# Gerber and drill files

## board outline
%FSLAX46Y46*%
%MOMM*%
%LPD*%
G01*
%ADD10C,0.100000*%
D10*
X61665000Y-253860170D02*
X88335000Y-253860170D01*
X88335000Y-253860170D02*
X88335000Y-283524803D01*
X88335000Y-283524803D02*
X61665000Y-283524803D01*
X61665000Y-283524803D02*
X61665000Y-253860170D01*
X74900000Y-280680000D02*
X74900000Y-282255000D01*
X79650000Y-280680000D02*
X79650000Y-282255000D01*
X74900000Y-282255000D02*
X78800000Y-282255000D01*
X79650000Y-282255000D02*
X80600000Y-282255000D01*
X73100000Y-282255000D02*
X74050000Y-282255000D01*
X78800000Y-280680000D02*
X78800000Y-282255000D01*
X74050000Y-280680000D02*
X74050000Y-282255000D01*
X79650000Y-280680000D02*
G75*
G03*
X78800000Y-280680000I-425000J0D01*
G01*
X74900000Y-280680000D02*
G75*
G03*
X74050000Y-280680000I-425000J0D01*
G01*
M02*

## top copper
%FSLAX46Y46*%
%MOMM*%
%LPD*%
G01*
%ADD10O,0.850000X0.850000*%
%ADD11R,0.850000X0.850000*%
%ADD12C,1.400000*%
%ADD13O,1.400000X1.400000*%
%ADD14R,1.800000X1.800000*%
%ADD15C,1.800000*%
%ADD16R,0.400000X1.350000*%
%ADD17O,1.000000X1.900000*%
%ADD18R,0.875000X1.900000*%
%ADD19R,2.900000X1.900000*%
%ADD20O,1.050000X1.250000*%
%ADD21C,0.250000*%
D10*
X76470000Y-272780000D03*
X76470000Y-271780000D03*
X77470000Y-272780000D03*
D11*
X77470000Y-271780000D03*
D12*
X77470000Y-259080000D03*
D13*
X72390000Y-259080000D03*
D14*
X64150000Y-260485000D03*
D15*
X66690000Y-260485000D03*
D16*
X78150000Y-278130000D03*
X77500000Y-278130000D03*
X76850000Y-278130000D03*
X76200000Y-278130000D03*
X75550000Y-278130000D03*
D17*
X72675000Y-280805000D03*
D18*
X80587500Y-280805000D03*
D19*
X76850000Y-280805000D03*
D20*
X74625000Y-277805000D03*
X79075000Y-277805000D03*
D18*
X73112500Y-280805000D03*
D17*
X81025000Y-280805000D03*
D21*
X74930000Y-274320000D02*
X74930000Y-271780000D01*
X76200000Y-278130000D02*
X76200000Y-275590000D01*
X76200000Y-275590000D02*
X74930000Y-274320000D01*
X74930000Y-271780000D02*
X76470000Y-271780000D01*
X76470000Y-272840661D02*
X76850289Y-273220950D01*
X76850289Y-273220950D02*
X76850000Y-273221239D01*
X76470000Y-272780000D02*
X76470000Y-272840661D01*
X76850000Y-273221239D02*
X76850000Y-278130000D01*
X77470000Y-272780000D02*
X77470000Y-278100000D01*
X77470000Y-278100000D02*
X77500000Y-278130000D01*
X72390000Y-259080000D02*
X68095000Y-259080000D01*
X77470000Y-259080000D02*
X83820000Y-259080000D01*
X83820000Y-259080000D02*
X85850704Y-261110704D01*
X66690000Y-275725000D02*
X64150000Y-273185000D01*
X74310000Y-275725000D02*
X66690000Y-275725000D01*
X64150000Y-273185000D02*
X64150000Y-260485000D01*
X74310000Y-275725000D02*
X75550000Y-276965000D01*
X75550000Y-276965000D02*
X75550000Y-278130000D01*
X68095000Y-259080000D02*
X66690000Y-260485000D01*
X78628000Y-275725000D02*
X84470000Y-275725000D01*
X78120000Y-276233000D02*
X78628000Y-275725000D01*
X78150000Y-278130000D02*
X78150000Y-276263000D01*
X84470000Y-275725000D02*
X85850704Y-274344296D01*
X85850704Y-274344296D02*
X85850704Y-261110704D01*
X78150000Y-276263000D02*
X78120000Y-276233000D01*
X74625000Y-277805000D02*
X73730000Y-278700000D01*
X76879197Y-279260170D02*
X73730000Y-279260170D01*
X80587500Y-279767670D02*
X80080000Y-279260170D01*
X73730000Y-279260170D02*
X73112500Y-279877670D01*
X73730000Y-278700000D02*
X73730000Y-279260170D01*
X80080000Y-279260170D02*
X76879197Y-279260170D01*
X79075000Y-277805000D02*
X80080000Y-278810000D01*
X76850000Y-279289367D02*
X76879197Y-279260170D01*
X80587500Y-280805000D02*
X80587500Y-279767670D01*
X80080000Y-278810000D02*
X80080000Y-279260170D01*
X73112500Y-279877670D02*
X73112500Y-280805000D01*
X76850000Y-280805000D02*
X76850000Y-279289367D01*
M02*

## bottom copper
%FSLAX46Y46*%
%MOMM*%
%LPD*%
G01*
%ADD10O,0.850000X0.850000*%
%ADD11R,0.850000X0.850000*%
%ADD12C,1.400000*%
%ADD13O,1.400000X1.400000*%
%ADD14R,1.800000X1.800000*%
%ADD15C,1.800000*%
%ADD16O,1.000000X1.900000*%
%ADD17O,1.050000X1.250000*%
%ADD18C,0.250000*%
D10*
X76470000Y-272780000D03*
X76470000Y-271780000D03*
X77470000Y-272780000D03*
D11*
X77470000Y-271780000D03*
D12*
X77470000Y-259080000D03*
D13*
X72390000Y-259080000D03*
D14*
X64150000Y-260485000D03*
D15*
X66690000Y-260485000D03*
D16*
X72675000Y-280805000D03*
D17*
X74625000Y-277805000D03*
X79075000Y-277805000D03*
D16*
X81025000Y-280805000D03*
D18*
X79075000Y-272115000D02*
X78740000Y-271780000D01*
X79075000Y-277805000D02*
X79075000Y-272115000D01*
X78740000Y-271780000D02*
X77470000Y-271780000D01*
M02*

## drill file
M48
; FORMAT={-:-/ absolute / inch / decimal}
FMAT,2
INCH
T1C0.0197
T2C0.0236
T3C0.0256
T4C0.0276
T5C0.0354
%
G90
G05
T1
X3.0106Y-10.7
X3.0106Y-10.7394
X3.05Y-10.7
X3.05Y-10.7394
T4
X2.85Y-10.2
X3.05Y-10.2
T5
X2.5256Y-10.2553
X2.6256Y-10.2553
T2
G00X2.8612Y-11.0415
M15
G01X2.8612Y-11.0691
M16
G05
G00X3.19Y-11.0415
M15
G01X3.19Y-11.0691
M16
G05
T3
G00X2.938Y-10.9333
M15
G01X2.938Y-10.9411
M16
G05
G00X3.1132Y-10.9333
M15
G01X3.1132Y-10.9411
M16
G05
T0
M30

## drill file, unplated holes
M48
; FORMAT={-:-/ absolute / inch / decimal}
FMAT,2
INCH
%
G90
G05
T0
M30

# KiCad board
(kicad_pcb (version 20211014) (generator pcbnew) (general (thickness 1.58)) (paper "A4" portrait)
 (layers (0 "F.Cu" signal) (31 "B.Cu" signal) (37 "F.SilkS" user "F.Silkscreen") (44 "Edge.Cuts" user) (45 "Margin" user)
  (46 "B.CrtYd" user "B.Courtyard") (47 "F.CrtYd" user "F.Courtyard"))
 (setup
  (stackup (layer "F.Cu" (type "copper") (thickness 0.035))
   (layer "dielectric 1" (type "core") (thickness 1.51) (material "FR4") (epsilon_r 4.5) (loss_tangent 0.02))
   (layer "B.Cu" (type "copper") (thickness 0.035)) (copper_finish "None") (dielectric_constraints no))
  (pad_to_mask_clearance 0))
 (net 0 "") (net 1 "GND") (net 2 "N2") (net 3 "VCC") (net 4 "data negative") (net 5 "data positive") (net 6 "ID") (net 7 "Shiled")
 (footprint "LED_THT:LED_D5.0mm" (layer "F.Cu") (at 64.15 260.485)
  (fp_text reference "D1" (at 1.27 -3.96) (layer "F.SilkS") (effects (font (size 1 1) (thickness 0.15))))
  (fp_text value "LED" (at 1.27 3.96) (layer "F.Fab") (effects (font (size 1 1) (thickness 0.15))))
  (pad "1" thru_hole rect (at 0 0) (size 1.8 1.8) (drill 0.9) (layers *.Cu *.Mask) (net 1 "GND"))
  (pad "2" thru_hole circle (at 2.54 0) (size 1.8 1.8) (drill 0.9) (layers *.Cu *.Mask) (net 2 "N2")))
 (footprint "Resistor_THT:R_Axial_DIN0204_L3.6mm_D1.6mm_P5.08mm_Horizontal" (layer "F.Cu") (at 77.47 259.08 180)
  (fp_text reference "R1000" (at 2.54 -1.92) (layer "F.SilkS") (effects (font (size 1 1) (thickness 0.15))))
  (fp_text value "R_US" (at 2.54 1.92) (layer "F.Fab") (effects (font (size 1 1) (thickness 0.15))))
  (pad "1" thru_hole circle (at 0 0 180) (size 1.4 1.4) (drill 0.7) (layers *.Cu *.Mask) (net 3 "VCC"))
  (pad "2" thru_hole oval (at 5.08 0 180) (size 1.4 1.4) (drill 0.7) (layers *.Cu *.Mask) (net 2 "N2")))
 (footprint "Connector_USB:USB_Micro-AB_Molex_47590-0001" (layer "F.Cu") (at 76.85 280.805)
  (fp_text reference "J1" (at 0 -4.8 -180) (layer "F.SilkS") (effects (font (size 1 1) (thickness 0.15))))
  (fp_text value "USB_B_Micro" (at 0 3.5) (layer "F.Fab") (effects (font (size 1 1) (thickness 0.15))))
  (fp_line (start -1.95 -0.125) (end -1.95 1.45) (layer "Edge.Cuts") (width 0.1))
  (fp_line (start 2.8 -0.125) (end 2.8 1.45) (layer "Edge.Cuts") (width 0.1))
  (fp_line (start -1.95 1.45) (end 1.95 1.45) (layer "Edge.Cuts") (width 0.1))
  (fp_line (start 2.8 1.45) (end 3.75 1.45) (layer "Edge.Cuts") (width 0.1))
  (fp_line (start -3.75 1.45) (end -2.8 1.45) (layer "Edge.Cuts") (width 0.1))
  (fp_line (start 1.95 -0.125) (end 1.95 1.45) (layer "Edge.Cuts") (width 0.1))
  (fp_line (start -2.8 -0.125) (end -2.8 1.45) (layer "Edge.Cuts") (width 0.1))
  (fp_arc (start 1.95 -0.125) (mid 2.375 -0.55) (end 2.8 -0.125) (layer "Edge.Cuts") (width 0.1))
  (fp_arc (start -2.8 -0.125) (mid -2.375 -0.55) (end -1.95 -0.125) (layer "Edge.Cuts") (width 0.1))
  (pad "" smd rect (at 3.5 0) (size 0.3 0.85) (layers "F.Paste"))
  (pad "" smd rect (at -3.5 0) (size 0.3 0.85) (layers "F.Paste"))
  (pad "1" smd rect (at 1.3 -2.675) (size 0.4 1.35) (layers "F.Cu" "F.Paste" "F.Mask") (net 3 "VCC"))
  (pad "2" smd rect (at 0.65 -2.675) (size 0.4 1.35) (layers "F.Cu" "F.Paste" "F.Mask") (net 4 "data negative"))
  (pad "3" smd rect (at 0 -2.675) (size 0.4 1.35) (layers "F.Cu" "F.Paste" "F.Mask") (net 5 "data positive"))
  (pad "4" smd rect (at -0.65 -2.675) (size 0.4 1.35) (layers "F.Cu" "F.Paste" "F.Mask") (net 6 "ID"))
  (pad "5" smd rect (at -1.3 -2.675) (size 0.4 1.35) (layers "F.Cu" "F.Paste" "F.Mask") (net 1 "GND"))
  (pad "6" thru_hole oval (at -4.175 0) (size 1 1.9) (drill oval 0.6 1.3) (layers *.Cu *.Mask) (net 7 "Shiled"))
  (pad "6" smd rect (at 3.7375 0) (size 0.875 1.9) (layers "F.Cu" "F.Mask") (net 7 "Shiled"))
  (pad "6" smd rect (at 0 0) (size 2.9 1.9) (layers "F.Cu" "F.Paste" "F.Mask") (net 7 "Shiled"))
  (pad "6" thru_hole oval (at -2.225 -3) (size 1.05 1.25) (drill oval 0.65 0.85) (layers *.Cu *.Mask) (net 7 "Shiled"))
  (pad "6" thru_hole oval (at 2.225 -3) (size 1.05 1.25) (drill oval 0.65 0.85) (layers *.Cu *.Mask) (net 7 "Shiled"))
  (pad "6" smd rect (at -3.7375 0) (size 0.875 1.9) (layers "F.Cu" "F.Mask") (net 7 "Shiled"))
  (pad "6" thru_hole oval (at 4.175 0) (size 1 1.9) (drill oval 0.6 1.3) (layers *.Cu *.Mask) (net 7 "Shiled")))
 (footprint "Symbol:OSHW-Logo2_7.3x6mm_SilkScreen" (layer "F.Cu") (at 66.11 280.53017)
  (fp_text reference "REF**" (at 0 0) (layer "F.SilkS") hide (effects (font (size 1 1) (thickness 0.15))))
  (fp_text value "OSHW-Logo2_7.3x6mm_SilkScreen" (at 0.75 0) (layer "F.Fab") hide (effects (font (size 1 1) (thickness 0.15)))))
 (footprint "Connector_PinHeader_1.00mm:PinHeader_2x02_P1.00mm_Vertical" (layer "F.Cu") (at 77.47 271.78 -90)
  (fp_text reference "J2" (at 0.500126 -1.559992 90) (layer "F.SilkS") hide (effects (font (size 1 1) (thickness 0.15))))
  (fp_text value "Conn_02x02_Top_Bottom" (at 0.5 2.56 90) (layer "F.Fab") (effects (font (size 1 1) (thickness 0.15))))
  (pad "1" thru_hole rect (at 0 0 270) (size 0.85 0.85) (drill 0.5) (layers *.Cu *.Mask) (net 7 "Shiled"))
  (pad "2" thru_hole oval (at 1 0 270) (size 0.85 0.85) (drill 0.5) (layers *.Cu *.Mask) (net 4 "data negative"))
  (pad "3" thru_hole oval (at 0 1 270) (size 0.85 0.85) (drill 0.5) (layers *.Cu *.Mask) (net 6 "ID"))
  (pad "4" thru_hole oval (at 1 1 270) (size 0.85 0.85) (drill 0.5) (layers *.Cu *.Mask) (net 5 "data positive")))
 (gr_rect (start 61.665 253.86017) (end 88.335 283.524803) (layer "Edge.Cuts") (width 0.1) (fill none))
 (segment (start 66.69 275.725) (end 64.15 273.185) (width 0.25) (layer "F.Cu") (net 1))
 (segment (start 74.31 275.725) (end 66.69 275.725) (width 0.25) (layer "F.Cu") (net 1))
 (segment (start 64.15 273.185) (end 64.15 260.485) (width 0.25) (layer "F.Cu") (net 1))
 (segment (start 74.31 275.725) (end 75.55 276.965) (width 0.25) (layer "F.Cu") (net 1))
 (segment (start 75.55 276.965) (end 75.55 278.13) (width 0.25) (layer "F.Cu") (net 1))
 (segment (start 72.39 259.08) (end 68.095 259.08) (width 0.25) (layer "F.Cu") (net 2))
 (segment (start 68.095 259.08) (end 66.69 260.485) (width 0.25) (layer "F.Cu") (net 2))
 (segment (start 78.628 275.725) (end 84.47 275.725) (width 0.25) (layer "F.Cu") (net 3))
 (segment (start 78.12 276.233) (end 78.628 275.725) (width 0.25) (layer "F.Cu") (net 3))
 (segment (start 78.15 278.13) (end 78.15 276.263) (width 0.25) (layer "F.Cu") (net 3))
 (segment (start 84.47 275.725) (end 85.850704 274.344296) (width 0.25) (layer "F.Cu") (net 3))
 (segment (start 85.850704 274.344296) (end 85.850704 261.110704) (width 0.25) (layer "F.Cu") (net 3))
 (segment (start 83.82 259.08) (end 85.850704 261.110704) (width 0.25) (layer "F.Cu") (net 3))
 (segment (start 77.47 259.08) (end 83.82 259.08) (width 0.25) (layer "F.Cu") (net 3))
 (segment (start 78.15 276.263) (end 78.12 276.233) (width 0.25) (layer "F.Cu") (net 3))
 (segment (start 77.47 278.1) (end 77.5 278.13) (width 0.25) (layer "F.Cu") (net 4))
 (segment (start 77.47 272.78) (end 77.47 278.1) (width 0.25) (layer "F.Cu") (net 4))
 (segment (start 76.47 272.840661) (end 76.850289 273.22095) (width 0.25) (layer "F.Cu") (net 5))
 (segment (start 76.850289 273.22095) (end 76.85 273.221239) (width 0.25) (layer "F.Cu") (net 5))
 (segment (start 76.47 272.78) (end 76.47 272.840661) (width 0.25) (layer "F.Cu") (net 5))
 (segment (start 76.85 273.221239) (end 76.85 278.13) (width 0.25) (layer "F.Cu") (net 5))
 (segment (start 76.2 278.13) (end 76.2 275.59) (width 0.25) (layer "F.Cu") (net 6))
 (segment (start 74.93 271.78) (end 76.47 271.78) (width 0.25) (layer "F.Cu") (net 6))
 (segment (start 74.93 274.32) (end 74.93 271.78) (width 0.25) (layer "F.Cu") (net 6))
 (segment (start 76.2 275.59) (end 74.93 274.32) (width 0.25) (layer "F.Cu") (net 6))
 (segment (start 74.625 277.805) (end 73.73 278.7) (width 0.25) (layer "F.Cu") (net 7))
 (segment (start 76.879197 279.26017) (end 73.73 279.26017) (width 0.25) (layer "F.Cu") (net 7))
 (segment (start 80.5875 279.76767) (end 80.08 279.26017) (width 0.25) (layer "F.Cu") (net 7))
 (segment (start 73.73 279.26017) (end 73.1125 279.87767) (width 0.25) (layer "F.Cu") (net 7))
 (segment (start 73.73 278.7) (end 73.73 279.26017) (width 0.25) (layer "F.Cu") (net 7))
 (segment (start 80.08 279.26017) (end 76.879197 279.26017) (width 0.25) (layer "F.Cu") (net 7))
 (segment (start 79.075 277.805) (end 80.08 278.81) (width 0.25) (layer "F.Cu") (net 7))
 (segment (start 76.85 279.289367) (end 76.879197 279.26017) (width 0.25) (layer "F.Cu") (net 7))
 (segment (start 80.5875 280.805) (end 80.5875 279.76767) (width 0.25) (layer "F.Cu") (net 7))
 (segment (start 80.08 278.81) (end 80.08 279.26017) (width 0.25) (layer "F.Cu") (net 7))
 (segment (start 73.1125 279.87767) (end 73.1125 280.805) (width 0.25) (layer "F.Cu") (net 7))
 (segment (start 76.85 280.805) (end 76.85 279.289367) (width 0.25) (layer "F.Cu") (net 7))
 (segment (start 78.74 271.78) (end 77.47 271.78) (width 0.25) (layer "B.Cu") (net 7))
 (segment (start 79.075 272.115) (end 78.74 271.78) (width 0.25) (layer "B.Cu") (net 7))
 (segment (start 79.075 277.805) (end 79.075 272.115) (width 0.25) (layer "B.Cu") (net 7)))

